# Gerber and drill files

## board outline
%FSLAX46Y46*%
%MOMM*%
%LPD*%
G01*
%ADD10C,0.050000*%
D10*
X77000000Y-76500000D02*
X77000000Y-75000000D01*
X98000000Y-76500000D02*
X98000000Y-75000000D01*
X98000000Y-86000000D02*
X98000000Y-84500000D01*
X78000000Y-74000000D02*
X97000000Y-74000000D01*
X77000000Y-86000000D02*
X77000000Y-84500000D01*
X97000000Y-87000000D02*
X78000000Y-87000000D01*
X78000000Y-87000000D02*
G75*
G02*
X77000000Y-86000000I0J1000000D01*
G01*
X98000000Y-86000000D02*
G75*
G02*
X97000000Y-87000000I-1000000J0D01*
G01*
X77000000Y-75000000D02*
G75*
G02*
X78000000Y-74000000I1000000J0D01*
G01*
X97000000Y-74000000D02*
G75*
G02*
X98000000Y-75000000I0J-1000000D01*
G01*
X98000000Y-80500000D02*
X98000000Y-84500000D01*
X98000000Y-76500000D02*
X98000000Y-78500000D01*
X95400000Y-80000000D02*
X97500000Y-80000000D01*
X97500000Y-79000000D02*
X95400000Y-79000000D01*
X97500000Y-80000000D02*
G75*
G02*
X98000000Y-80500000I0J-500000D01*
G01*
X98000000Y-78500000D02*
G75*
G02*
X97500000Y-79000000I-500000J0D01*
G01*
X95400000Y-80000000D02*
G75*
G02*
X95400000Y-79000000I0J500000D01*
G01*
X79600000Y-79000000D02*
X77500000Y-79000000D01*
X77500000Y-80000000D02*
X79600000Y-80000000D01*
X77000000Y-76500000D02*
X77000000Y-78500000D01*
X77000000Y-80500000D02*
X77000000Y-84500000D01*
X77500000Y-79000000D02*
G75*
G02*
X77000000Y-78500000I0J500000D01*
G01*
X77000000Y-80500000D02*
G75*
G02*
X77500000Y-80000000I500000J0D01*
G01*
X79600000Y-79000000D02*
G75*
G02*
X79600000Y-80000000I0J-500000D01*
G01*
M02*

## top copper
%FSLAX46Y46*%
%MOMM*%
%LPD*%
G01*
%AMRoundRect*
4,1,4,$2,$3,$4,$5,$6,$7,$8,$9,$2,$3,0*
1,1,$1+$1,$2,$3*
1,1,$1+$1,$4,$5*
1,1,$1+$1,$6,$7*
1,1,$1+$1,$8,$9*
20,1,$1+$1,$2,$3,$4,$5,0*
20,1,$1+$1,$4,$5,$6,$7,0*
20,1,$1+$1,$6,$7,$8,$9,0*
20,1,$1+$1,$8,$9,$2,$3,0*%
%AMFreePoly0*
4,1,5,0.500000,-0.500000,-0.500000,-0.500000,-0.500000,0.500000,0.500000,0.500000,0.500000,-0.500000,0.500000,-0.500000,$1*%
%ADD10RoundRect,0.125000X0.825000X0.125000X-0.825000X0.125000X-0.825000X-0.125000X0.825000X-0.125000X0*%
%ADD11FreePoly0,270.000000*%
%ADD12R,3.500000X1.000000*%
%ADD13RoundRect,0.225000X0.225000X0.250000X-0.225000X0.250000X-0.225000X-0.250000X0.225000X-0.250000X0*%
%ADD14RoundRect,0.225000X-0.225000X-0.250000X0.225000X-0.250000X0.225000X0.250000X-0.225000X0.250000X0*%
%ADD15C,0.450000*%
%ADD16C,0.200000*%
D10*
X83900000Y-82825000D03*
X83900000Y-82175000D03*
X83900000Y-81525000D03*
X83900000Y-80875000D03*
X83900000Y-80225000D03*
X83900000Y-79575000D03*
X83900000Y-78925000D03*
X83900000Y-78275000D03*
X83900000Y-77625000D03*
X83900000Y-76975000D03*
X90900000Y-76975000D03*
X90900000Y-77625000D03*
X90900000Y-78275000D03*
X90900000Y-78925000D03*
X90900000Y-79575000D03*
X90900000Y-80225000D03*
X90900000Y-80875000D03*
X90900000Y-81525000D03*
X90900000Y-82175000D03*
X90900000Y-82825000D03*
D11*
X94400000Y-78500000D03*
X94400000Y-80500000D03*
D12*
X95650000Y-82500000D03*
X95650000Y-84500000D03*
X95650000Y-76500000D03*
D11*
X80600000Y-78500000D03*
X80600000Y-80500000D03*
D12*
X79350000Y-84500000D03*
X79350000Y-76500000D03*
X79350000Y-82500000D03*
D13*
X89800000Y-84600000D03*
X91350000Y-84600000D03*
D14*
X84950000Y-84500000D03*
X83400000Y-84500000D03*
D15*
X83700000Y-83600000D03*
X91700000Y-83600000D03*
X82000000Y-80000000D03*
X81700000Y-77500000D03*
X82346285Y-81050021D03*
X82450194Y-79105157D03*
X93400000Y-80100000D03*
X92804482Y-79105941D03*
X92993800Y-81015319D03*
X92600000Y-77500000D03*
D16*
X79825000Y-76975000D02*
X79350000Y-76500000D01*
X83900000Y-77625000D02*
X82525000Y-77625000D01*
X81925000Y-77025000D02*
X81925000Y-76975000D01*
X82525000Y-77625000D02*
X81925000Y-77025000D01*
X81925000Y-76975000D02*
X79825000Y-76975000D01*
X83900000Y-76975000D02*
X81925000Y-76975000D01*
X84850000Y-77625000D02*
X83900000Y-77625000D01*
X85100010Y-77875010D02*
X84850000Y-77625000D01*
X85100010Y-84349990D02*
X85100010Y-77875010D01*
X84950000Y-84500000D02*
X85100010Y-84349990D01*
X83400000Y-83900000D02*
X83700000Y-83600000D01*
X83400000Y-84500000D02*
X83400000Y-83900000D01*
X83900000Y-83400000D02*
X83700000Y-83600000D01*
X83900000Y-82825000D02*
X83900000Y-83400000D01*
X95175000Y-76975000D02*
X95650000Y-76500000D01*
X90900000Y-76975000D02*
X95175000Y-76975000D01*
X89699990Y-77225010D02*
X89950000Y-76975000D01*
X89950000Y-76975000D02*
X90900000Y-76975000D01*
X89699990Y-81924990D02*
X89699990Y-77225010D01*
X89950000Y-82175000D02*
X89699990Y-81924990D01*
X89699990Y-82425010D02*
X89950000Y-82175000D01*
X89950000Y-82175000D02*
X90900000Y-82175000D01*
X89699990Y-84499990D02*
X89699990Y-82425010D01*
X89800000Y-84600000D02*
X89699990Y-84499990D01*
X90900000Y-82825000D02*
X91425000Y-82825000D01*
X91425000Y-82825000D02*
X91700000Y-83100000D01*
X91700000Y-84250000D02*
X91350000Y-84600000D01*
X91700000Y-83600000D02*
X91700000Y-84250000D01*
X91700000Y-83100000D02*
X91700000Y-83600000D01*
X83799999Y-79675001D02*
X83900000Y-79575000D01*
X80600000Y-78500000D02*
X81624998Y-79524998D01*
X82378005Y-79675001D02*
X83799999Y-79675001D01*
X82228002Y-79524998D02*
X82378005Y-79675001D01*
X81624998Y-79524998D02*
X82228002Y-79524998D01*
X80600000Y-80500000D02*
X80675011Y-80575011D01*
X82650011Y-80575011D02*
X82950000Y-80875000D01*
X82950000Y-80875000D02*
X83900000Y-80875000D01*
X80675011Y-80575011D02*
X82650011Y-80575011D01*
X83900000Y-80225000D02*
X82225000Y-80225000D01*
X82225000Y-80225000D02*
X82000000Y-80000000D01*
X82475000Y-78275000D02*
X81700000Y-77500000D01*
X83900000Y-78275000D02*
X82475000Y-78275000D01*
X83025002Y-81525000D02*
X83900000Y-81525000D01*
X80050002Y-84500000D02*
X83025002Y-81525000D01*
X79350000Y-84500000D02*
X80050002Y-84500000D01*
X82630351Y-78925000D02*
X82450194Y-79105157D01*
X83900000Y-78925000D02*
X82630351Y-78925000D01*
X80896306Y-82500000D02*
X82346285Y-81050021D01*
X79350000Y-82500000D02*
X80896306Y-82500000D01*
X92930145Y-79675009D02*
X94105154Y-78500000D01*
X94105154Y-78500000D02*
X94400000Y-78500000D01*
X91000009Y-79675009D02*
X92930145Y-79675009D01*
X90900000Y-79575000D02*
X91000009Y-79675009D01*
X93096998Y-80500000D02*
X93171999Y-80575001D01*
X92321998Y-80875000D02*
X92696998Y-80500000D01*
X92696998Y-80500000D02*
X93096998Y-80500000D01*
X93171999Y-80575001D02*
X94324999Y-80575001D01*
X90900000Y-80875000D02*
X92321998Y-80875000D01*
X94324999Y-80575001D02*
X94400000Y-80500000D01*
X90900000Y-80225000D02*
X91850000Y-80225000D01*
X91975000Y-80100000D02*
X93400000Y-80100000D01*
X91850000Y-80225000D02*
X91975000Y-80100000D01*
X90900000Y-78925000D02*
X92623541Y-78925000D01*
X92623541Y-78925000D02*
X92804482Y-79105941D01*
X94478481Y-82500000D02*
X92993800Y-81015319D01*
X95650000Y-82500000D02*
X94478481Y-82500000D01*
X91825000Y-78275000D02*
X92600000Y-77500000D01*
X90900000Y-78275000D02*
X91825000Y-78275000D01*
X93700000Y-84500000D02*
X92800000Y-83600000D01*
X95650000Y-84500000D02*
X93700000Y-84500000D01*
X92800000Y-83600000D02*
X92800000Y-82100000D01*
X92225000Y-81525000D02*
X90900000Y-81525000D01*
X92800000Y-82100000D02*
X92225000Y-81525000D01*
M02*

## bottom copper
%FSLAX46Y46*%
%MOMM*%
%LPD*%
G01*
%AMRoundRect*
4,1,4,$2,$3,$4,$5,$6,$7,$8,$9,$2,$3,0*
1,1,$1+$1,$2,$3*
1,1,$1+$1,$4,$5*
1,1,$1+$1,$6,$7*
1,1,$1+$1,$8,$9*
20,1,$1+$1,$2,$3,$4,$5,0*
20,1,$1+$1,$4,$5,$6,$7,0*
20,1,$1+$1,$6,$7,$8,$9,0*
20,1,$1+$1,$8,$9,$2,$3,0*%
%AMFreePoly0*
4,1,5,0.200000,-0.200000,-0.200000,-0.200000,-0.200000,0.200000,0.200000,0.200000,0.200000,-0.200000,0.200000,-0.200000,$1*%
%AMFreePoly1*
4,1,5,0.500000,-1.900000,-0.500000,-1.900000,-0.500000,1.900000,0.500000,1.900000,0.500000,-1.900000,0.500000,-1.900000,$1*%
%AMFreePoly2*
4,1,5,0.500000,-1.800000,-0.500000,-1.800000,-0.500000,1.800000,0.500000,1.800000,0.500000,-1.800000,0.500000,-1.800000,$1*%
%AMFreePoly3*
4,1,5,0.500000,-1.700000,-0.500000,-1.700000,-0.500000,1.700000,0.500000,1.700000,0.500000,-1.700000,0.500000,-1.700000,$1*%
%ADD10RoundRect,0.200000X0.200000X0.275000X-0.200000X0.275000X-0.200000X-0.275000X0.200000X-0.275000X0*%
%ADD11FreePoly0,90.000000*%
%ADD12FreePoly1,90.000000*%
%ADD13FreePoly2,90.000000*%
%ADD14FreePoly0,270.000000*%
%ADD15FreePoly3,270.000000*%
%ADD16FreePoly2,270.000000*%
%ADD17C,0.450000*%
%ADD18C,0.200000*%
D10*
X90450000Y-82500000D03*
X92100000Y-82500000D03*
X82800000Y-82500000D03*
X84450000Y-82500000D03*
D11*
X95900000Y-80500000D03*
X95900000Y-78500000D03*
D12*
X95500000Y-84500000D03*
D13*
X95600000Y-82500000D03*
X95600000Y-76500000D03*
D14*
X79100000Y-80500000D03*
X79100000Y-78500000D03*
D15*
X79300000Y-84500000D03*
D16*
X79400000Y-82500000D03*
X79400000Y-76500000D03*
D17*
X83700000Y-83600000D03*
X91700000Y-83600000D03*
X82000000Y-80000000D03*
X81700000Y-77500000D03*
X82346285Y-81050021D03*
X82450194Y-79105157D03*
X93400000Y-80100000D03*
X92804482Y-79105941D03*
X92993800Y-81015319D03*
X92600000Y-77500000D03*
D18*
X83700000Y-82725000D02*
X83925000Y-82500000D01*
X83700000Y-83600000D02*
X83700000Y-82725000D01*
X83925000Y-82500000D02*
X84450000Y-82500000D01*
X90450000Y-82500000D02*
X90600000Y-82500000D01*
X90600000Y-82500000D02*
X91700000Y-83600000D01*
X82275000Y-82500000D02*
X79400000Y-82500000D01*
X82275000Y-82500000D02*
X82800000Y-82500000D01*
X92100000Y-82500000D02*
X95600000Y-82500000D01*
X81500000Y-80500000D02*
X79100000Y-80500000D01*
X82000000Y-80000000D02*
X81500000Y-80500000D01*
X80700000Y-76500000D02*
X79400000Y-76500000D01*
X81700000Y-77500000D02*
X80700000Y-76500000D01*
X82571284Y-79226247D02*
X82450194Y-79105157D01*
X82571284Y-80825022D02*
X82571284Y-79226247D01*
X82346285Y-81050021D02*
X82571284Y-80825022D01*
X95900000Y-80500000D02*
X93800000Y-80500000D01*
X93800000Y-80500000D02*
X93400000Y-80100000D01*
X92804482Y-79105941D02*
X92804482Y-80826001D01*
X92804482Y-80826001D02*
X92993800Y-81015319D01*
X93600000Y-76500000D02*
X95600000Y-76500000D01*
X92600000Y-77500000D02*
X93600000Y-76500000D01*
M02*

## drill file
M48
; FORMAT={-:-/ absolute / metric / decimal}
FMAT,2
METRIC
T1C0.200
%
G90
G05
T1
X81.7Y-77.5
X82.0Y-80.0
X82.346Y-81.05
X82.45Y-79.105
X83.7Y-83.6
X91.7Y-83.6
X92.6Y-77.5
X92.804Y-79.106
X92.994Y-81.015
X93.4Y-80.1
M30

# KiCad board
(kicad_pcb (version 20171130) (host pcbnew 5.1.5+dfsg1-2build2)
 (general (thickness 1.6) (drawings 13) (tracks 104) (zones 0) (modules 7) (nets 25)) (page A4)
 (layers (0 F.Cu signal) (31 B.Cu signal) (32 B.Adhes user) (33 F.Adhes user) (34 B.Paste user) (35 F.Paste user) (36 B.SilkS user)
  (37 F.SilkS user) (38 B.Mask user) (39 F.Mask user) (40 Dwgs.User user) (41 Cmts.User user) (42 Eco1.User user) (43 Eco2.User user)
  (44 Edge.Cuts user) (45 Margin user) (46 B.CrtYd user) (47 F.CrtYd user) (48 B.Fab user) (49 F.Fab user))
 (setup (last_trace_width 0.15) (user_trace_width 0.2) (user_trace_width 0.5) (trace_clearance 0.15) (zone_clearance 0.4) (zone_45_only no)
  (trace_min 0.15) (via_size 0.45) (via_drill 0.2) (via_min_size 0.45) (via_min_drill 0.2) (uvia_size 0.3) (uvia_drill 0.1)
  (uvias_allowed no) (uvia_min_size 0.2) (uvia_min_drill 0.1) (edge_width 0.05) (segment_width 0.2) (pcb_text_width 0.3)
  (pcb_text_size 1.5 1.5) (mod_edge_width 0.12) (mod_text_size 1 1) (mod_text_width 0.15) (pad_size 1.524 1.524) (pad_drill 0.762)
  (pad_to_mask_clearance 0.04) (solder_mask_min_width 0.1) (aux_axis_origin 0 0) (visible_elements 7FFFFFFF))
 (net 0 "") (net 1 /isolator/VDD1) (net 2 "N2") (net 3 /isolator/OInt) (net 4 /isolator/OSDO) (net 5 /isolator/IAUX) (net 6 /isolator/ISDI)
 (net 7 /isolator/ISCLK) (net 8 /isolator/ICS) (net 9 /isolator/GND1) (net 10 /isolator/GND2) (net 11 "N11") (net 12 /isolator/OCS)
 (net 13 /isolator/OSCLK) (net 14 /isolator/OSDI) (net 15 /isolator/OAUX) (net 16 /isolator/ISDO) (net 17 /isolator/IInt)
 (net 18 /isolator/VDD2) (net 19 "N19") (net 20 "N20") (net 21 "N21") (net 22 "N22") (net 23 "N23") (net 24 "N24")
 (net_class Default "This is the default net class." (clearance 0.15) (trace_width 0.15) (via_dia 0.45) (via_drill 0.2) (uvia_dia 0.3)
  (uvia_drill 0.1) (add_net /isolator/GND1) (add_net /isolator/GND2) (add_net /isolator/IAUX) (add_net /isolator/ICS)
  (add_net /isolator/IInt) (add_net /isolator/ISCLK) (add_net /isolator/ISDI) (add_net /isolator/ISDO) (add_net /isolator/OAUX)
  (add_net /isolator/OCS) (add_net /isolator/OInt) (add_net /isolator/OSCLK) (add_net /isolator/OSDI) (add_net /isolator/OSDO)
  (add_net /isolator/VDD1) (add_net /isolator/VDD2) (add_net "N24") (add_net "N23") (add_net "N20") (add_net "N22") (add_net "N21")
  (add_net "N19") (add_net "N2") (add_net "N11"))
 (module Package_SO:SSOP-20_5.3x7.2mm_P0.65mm (layer F.Cu) (at 87.4 79.9 180)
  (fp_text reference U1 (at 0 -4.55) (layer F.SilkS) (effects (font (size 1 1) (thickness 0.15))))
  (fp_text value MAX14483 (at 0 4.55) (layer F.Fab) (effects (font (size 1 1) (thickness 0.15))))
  (pad 20 smd roundrect (at 3.5 -2.925 180) (size 1.9 0.5) (layers F.Cu F.Paste F.Mask) (roundrect_rratio 0.25) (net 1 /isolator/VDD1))
  (pad 19 smd roundrect (at 3.5 -2.275 180) (size 1.9 0.5) (layers F.Cu F.Paste F.Mask) (roundrect_rratio 0.25) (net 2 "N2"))
  (pad 18 smd roundrect (at 3.5 -1.625 180) (size 1.9 0.5) (layers F.Cu F.Paste F.Mask) (roundrect_rratio 0.25) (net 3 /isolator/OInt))
  (pad 17 smd roundrect (at 3.5 -0.975 180) (size 1.9 0.5) (layers F.Cu F.Paste F.Mask) (roundrect_rratio 0.25) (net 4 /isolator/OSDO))
  (pad 16 smd roundrect (at 3.5 -0.325 180) (size 1.9 0.5) (layers F.Cu F.Paste F.Mask) (roundrect_rratio 0.25) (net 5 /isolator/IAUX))
  (pad 15 smd roundrect (at 3.5 0.325 180) (size 1.9 0.5) (layers F.Cu F.Paste F.Mask) (roundrect_rratio 0.25) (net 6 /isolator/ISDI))
  (pad 14 smd roundrect (at 3.5 0.975 180) (size 1.9 0.5) (layers F.Cu F.Paste F.Mask) (roundrect_rratio 0.25) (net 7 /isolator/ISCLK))
  (pad 13 smd roundrect (at 3.5 1.625 180) (size 1.9 0.5) (layers F.Cu F.Paste F.Mask) (roundrect_rratio 0.25) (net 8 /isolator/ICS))
  (pad 12 smd roundrect (at 3.5 2.275 180) (size 1.9 0.5) (layers F.Cu F.Paste F.Mask) (roundrect_rratio 0.25) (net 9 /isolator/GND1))
  (pad 11 smd roundrect (at 3.5 2.925 180) (size 1.9 0.5) (layers F.Cu F.Paste F.Mask) (roundrect_rratio 0.25) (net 9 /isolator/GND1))
  (pad 10 smd roundrect (at -3.5 2.925 180) (size 1.9 0.5) (layers F.Cu F.Paste F.Mask) (roundrect_rratio 0.25) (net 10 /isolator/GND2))
  (pad 9 smd roundrect (at -3.5 2.275 180) (size 1.9 0.5) (layers F.Cu F.Paste F.Mask) (roundrect_rratio 0.25) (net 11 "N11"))
  (pad 8 smd roundrect (at -3.5 1.625 180) (size 1.9 0.5) (layers F.Cu F.Paste F.Mask) (roundrect_rratio 0.25) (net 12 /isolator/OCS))
  (pad 7 smd roundrect (at -3.5 0.975 180) (size 1.9 0.5) (layers F.Cu F.Paste F.Mask) (roundrect_rratio 0.25) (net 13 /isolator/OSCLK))
  (pad 6 smd roundrect (at -3.5 0.325 180) (size 1.9 0.5) (layers F.Cu F.Paste F.Mask) (roundrect_rratio 0.25) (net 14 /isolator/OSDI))
  (pad 5 smd roundrect (at -3.5 -0.325 180) (size 1.9 0.5) (layers F.Cu F.Paste F.Mask) (roundrect_rratio 0.25) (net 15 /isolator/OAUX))
  (pad 4 smd roundrect (at -3.5 -0.975 180) (size 1.9 0.5) (layers F.Cu F.Paste F.Mask) (roundrect_rratio 0.25) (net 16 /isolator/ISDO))
  (pad 3 smd roundrect (at -3.5 -1.625 180) (size 1.9 0.5) (layers F.Cu F.Paste F.Mask) (roundrect_rratio 0.25) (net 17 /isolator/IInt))
  (pad 2 smd roundrect (at -3.5 -2.275 180) (size 1.9 0.5) (layers F.Cu F.Paste F.Mask) (roundrect_rratio 0.25) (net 10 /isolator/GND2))
  (pad 1 smd roundrect (at -3.5 -2.925 180) (size 1.9 0.5) (layers F.Cu F.Paste F.Mask) (roundrect_rratio 0.25) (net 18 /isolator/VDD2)))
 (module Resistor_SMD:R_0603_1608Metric (layer B.Cu) (at 91.275 82.5 180)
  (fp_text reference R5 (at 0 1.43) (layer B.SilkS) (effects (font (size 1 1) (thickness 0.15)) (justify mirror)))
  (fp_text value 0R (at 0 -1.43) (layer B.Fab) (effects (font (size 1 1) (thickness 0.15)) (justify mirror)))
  (pad 2 smd roundrect (at 0.825 0 180) (size 0.8 0.95) (layers B.Cu B.Paste B.Mask) (roundrect_rratio 0.25) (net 18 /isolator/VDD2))
  (pad 1 smd roundrect (at -0.825 0 180) (size 0.8 0.95) (layers B.Cu B.Paste B.Mask) (roundrect_rratio 0.25) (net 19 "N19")))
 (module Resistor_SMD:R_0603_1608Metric (layer B.Cu) (at 83.625 82.5 180)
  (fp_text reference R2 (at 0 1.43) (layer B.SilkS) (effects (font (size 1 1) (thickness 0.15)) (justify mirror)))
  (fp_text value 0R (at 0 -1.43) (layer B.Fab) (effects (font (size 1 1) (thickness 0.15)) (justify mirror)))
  (pad 2 smd roundrect (at 0.825 0 180) (size 0.8 0.95) (layers B.Cu B.Paste B.Mask) (roundrect_rratio 0.25) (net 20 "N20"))
  (pad 1 smd roundrect (at -0.825 0 180) (size 0.8 0.95) (layers B.Cu B.Paste B.Mask) (roundrect_rratio 0.25) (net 1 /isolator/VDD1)))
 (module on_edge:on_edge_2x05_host (layer F.Cu) (at 98 80.5 270)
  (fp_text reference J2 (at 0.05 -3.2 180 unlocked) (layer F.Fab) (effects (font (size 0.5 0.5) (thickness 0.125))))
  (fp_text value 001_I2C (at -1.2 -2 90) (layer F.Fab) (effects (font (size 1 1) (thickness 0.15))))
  (fp_line (start 0 0) (end 4 0) (layer Edge.Cuts) (width 0.05))
  (fp_line (start -4 0) (end -2 0) (layer Edge.Cuts) (width 0.05))
  (fp_line (start -0.5 2.6) (end -0.5 0.5) (layer Edge.Cuts) (width 0.05))
  (fp_line (start -1.5 0.5) (end -1.5 2.6) (layer Edge.Cuts) (width 0.05))
  (fp_arc (start 0 0.5) (end 0 0) (angle -90) (layer Edge.Cuts) (width 0.05))
  (fp_arc (start -2 0.5) (end -1.5 0.5) (angle -90) (layer Edge.Cuts) (width 0.05))
  (fp_arc (start -1 2.6) (end -1.5 2.6) (angle -180) (layer Edge.Cuts) (width 0.05))
  (pad 2 smd custom (at -2 3.6 270) (size 1 1) (layers F.Cu F.Mask) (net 14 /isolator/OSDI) (zone_connect 0)
   (options (clearance outline) (anchor rect)) (primitives))
  (pad 3 smd custom (at 0 3.6 270) (size 1 1) (layers F.Cu F.Mask) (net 16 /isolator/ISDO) (zone_connect 0)
   (options (clearance outline) (anchor rect)) (primitives))
  (pad 8 smd custom (at 0 2.1 90) (size 0.4 0.4) (layers B.Cu B.Mask) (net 15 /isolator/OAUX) (zone_connect 0)
   (options (clearance outline) (anchor rect)) (primitives))
  (pad 7 smd custom (at -2 2.1 90) (size 0.4 0.4) (layers B.Cu B.Mask) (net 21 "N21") (zone_connect 0)
   (options (clearance outline) (anchor rect)) (primitives))
  (pad 4 smd rect (at 2 2.35 270) (size 1 3.5) (layers F.Cu F.Mask) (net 13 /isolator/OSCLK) (zone_connect 0))
  (pad 10 smd custom (at 4 2.5 90) (size 1 3.8) (layers B.Cu B.Mask) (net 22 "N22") (zone_connect 0)
   (options (clearance outline) (anchor rect)) (primitives))
  (pad 9 smd custom (at 2 2.4 90) (size 1 3.6) (layers B.Cu B.Mask) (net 19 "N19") (zone_connect 0)
   (options (clearance outline) (anchor rect)) (primitives))
  (pad 6 smd custom (at -4 2.4 90) (size 1 3.6) (layers B.Cu B.Mask) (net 12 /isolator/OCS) (zone_connect 0)
   (options (clearance outline) (anchor rect)) (primitives))
  (pad 5 smd rect (at 4 2.35 270) (size 1 3.5) (layers F.Cu F.Mask) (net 17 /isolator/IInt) (zone_connect 0))
  (pad 1 smd rect (at -4 2.35 270) (size 1 3.5) (layers F.Cu F.Mask) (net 10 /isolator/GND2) (zone_connect 0)))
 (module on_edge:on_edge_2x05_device (layer F.Cu) (at 77 80.5 270)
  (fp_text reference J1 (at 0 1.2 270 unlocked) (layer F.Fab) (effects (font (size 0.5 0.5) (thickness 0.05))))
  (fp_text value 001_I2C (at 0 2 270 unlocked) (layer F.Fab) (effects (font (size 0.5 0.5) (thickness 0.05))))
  (fp_line (start -1.5 -2.6) (end -1.5 -0.5) (layer Edge.Cuts) (width 0.05))
  (fp_line (start -0.5 -0.5) (end -0.5 -2.6) (layer Edge.Cuts) (width 0.05))
  (fp_line (start -4 0) (end -2 0) (layer Edge.Cuts) (width 0.05))
  (fp_line (start 0 0) (end 4 0) (layer Edge.Cuts) (width 0.05))
  (fp_arc (start -2 -0.5) (end -2 0) (angle -90) (layer Edge.Cuts) (width 0.05))
  (fp_arc (start 0 -0.5) (end -0.5 -0.5) (angle -90) (layer Edge.Cuts) (width 0.05))
  (fp_arc (start -1 -2.6) (end -0.5 -2.6) (angle -180) (layer Edge.Cuts) (width 0.05))
  (pad 2 smd custom (at -2 -3.6 270) (size 1 1) (layers F.Cu F.Mask) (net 6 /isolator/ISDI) (zone_connect 0)
   (options (clearance outline) (anchor rect)) (primitives))
  (pad 3 smd custom (at 0 -3.6 270) (size 1 1) (layers F.Cu F.Mask) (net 4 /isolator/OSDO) (zone_connect 0)
   (options (clearance outline) (anchor rect)) (primitives))
  (pad 8 smd custom (at 0 -2.1 270) (size 0.4 0.4) (layers B.Cu B.Mask) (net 5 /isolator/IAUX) (zone_connect 0)
   (options (clearance outline) (anchor rect)) (primitives))
  (pad 7 smd custom (at -2 -2.1 270) (size 0.4 0.4) (layers B.Cu B.Mask) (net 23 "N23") (zone_connect 0)
   (options (clearance outline) (anchor rect)) (primitives))
  (pad 10 smd custom (at 4 -2.3 270) (size 1 3.4) (layers B.Cu B.Mask) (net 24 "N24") (zone_connect 0)
   (options (clearance outline) (anchor rect)) (primitives))
  (pad 9 smd custom (at 2 -2.4 270) (size 1 3.6) (layers B.Cu B.Mask) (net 20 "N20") (zone_connect 0)
   (options (clearance outline) (anchor rect)) (primitives))
  (pad 6 smd custom (at -4 -2.4 270) (size 1 3.6) (layers B.Cu B.Mask) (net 8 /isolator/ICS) (zone_connect 0)
   (options (clearance outline) (anchor rect)) (primitives))
  (pad 5 smd rect (at 4 -2.35 90) (size 1 3.5) (layers F.Cu F.Mask) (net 3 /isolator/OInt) (zone_connect 0))
  (pad 1 smd rect (at -4 -2.35 90) (size 1 3.5) (layers F.Cu F.Mask) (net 9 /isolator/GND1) (zone_connect 0))
  (pad 4 smd rect (at 2 -2.35 90) (size 1 3.5) (layers F.Cu F.Mask) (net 7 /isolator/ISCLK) (zone_connect 0)))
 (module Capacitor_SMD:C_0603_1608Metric (layer F.Cu) (at 90.575 84.6 180)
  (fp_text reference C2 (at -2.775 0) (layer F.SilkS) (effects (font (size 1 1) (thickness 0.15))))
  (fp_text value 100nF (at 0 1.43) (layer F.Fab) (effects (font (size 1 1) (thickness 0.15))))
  (pad 2 smd roundrect (at 0.775 0 180) (size 0.9 0.95) (layers F.Cu F.Paste F.Mask) (roundrect_rratio 0.25) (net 10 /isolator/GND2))
  (pad 1 smd roundrect (at -0.775 0 180) (size 0.9 0.95) (layers F.Cu F.Paste F.Mask) (roundrect_rratio 0.25) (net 18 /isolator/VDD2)))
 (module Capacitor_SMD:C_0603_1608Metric (layer F.Cu) (at 84.175 84.5)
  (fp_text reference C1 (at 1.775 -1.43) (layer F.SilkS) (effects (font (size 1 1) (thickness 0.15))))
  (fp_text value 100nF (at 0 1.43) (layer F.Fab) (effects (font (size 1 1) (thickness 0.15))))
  (pad 2 smd roundrect (at 0.775 0) (size 0.9 0.95) (layers F.Cu F.Paste F.Mask) (roundrect_rratio 0.25) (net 9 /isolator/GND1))
  (pad 1 smd roundrect (at -0.775 0) (size 0.9 0.95) (layers F.Cu F.Paste F.Mask) (roundrect_rratio 0.25) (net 1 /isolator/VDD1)))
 (gr_line (start 77 76.5) (end 77 75) (layer Edge.Cuts) (width 0.05))
 (gr_line (start 98 76.5) (end 98 75) (layer Edge.Cuts) (width 0.05))
 (gr_line (start 98 86) (end 98 84.5) (layer Edge.Cuts) (width 0.05))
 (gr_line (start 78 74) (end 97 74) (layer Edge.Cuts) (width 0.05))
 (gr_line (start 77 86) (end 77 84.5) (layer Edge.Cuts) (width 0.05))
 (gr_line (start 97 87) (end 78 87) (layer Edge.Cuts) (width 0.05))
 (gr_arc (start 78 86) (end 77 86) (angle -90) (layer Edge.Cuts) (width 0.05))
 (gr_arc (start 97 86) (end 97 87) (angle -90) (layer Edge.Cuts) (width 0.05))
 (gr_arc (start 78 75) (end 78 74) (angle -90) (layer Edge.Cuts) (width 0.05))
 (gr_arc (start 97 75) (end 98 75) (angle -90) (layer Edge.Cuts) (width 0.05))
 (segment (start 79.825 76.975) (end 79.35 76.5) (width 0.2) (layer F.Cu) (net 9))
 (segment (start 83.9 77.625) (end 82.525 77.625) (width 0.2) (layer F.Cu) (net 9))
 (segment (start 81.925 77.025) (end 81.925 76.975) (width 0.2) (layer F.Cu) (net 9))
 (segment (start 82.525 77.625) (end 81.925 77.025) (width 0.2) (layer F.Cu) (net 9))
 (segment (start 81.925 76.975) (end 79.825 76.975) (width 0.2) (layer F.Cu) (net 9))
 (segment (start 83.9 76.975) (end 81.925 76.975) (width 0.2) (layer F.Cu) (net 9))
 (segment (start 84.85 77.625) (end 83.9 77.625) (width 0.2) (layer F.Cu) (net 9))
 (segment (start 85.10001 77.87501) (end 84.85 77.625) (width 0.2) (layer F.Cu) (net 9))
 (segment (start 85.10001 84.34999) (end 85.10001 77.87501) (width 0.2) (layer F.Cu) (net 9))
 (segment (start 84.95 84.5) (end 85.10001 84.34999) (width 0.2) (layer F.Cu) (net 9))
 (via (at 83.7 83.6) (size 0.45) (drill 0.2) (layers F.Cu B.Cu) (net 1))
 (segment (start 83.4 83.9) (end 83.7 83.6) (width 0.2) (layer F.Cu) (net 1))
 (segment (start 83.4 84.5) (end 83.4 83.9) (width 0.2) (layer F.Cu) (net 1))
 (segment (start 83.7 82.725) (end 83.925 82.5) (width 0.2) (layer B.Cu) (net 1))
 (segment (start 83.7 83.6) (end 83.7 82.725) (width 0.2) (layer B.Cu) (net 1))
 (segment (start 83.9 83.4) (end 83.7 83.6) (width 0.2) (layer F.Cu) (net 1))
 (segment (start 83.9 82.825) (end 83.9 83.4) (width 0.2) (layer F.Cu) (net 1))
 (segment (start 83.925 82.5) (end 84.45 82.5) (width 0.2) (layer B.Cu) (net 1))
 (segment (start 95.175 76.975) (end 95.65 76.5) (width 0.2) (layer F.Cu) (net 10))
 (segment (start 90.9 76.975) (end 95.175 76.975) (width 0.2) (layer F.Cu) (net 10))
 (segment (start 89.69999 77.22501) (end 89.95 76.975) (width 0.2) (layer F.Cu) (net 10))
 (segment (start 89.95 76.975) (end 90.9 76.975) (width 0.2) (layer F.Cu) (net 10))
 (segment (start 89.69999 81.92499) (end 89.69999 77.22501) (width 0.2) (layer F.Cu) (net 10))
 (segment (start 89.95 82.175) (end 89.69999 81.92499) (width 0.2) (layer F.Cu) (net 10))
 (segment (start 89.69999 82.42501) (end 89.95 82.175) (width 0.2) (layer F.Cu) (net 10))
 (segment (start 89.95 82.175) (end 90.9 82.175) (width 0.2) (layer F.Cu) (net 10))
 (segment (start 89.69999 84.49999) (end 89.69999 82.42501) (width 0.2) (layer F.Cu) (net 10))
 (segment (start 89.8 84.6) (end 89.69999 84.49999) (width 0.2) (layer F.Cu) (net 10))
 (segment (start 90.9 82.825) (end 91.425 82.825) (width 0.2) (layer F.Cu) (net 18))
 (segment (start 91.425 82.825) (end 91.7 83.1) (width 0.2) (layer F.Cu) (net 18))
 (segment (start 91.7 84.25) (end 91.35 84.6) (width 0.2) (layer F.Cu) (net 18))
 (via (at 91.7 83.6) (size 0.45) (drill 0.2) (layers F.Cu B.Cu) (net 18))
 (segment (start 90.45 82.5) (end 90.6 82.5) (width 0.2) (layer B.Cu) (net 18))
 (segment (start 91.7 83.6) (end 91.7 84.25) (width 0.2) (layer F.Cu) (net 18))
 (segment (start 90.6 82.5) (end 91.7 83.6) (width 0.2) (layer B.Cu) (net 18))
 (segment (start 91.7 83.1) (end 91.7 83.6) (width 0.2) (layer F.Cu) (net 18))
 (segment (start 82.275 82.5) (end 79.4 82.5) (width 0.2) (layer B.Cu) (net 20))
 (segment (start 82.275 82.5) (end 82.8 82.5) (width 0.2) (layer B.Cu) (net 20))
 (segment (start 92.1 82.5) (end 95.6 82.5) (width 0.2) (layer B.Cu) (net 19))
 (segment (start 83.799999 79.675001) (end 83.9 79.575) (width 0.2) (layer F.Cu) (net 6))
 (segment (start 80.6 78.5) (end 81.624998 79.524998) (width 0.2) (layer F.Cu) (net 6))
 (segment (start 82.378005 79.675001) (end 83.799999 79.675001) (width 0.2) (layer F.Cu) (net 6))
 (segment (start 82.228002 79.524998) (end 82.378005 79.675001) (width 0.2) (layer F.Cu) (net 6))
 (segment (start 81.624998 79.524998) (end 82.228002 79.524998) (width 0.2) (layer F.Cu) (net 6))
 (segment (start 80.6 80.5) (end 80.675011 80.575011) (width 0.2) (layer F.Cu) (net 4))
 (segment (start 82.650011 80.575011) (end 82.95 80.875) (width 0.2) (layer F.Cu) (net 4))
 (segment (start 82.95 80.875) (end 83.9 80.875) (width 0.2) (layer F.Cu) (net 4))
 (segment (start 80.675011 80.575011) (end 82.650011 80.575011) (width 0.2) (layer F.Cu) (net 4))
 (segment (start 83.9 80.225) (end 82.225 80.225) (width 0.2) (layer F.Cu) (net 5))
 (via (at 82 80) (size 0.45) (drill 0.2) (layers F.Cu B.Cu) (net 5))
 (segment (start 82.225 80.225) (end 82 80) (width 0.2) (layer F.Cu) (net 5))
 (segment (start 81.5 80.5) (end 79.1 80.5) (width 0.2) (layer B.Cu) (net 5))
 (segment (start 82 80) (end 81.5 80.5) (width 0.2) (layer B.Cu) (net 5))
 (via (at 81.7 77.5) (size 0.45) (drill 0.2) (layers F.Cu B.Cu) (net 8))
 (segment (start 82.475 78.275) (end 81.7 77.5) (width 0.2) (layer F.Cu) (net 8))
 (segment (start 83.9 78.275) (end 82.475 78.275) (width 0.2) (layer F.Cu) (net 8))
 (segment (start 80.7 76.5) (end 79.4 76.5) (width 0.2) (layer B.Cu) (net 8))
 (segment (start 81.7 77.5) (end 80.7 76.5) (width 0.2) (layer B.Cu) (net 8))
 (segment (start 83.025002 81.525) (end 83.9 81.525) (width 0.2) (layer F.Cu) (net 3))
 (segment (start 80.050002 84.5) (end 83.025002 81.525) (width 0.2) (layer F.Cu) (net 3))
 (segment (start 79.35 84.5) (end 80.050002 84.5) (width 0.2) (layer F.Cu) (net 3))
 (via (at 82.346285 81.050021) (size 0.45) (drill 0.2) (layers F.Cu B.Cu) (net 7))
 (segment (start 82.571284 79.226247) (end 82.450194 79.105157) (width 0.2) (layer B.Cu) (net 7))
 (segment (start 82.571284 80.825022) (end 82.571284 79.226247) (width 0.2) (layer B.Cu) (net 7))
 (segment (start 82.346285 81.050021) (end 82.571284 80.825022) (width 0.2) (layer B.Cu) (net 7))
 (segment (start 82.630351 78.925) (end 82.450194 79.105157) (width 0.2) (layer F.Cu) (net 7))
 (segment (start 83.9 78.925) (end 82.630351 78.925) (width 0.2) (layer F.Cu) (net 7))
 (via (at 82.450194 79.105157) (size 0.45) (drill 0.2) (layers F.Cu B.Cu) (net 7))
 (segment (start 80.896306 82.5) (end 82.346285 81.050021) (width 0.2) (layer F.Cu) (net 7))
 (segment (start 79.35 82.5) (end 80.896306 82.5) (width 0.2) (layer F.Cu) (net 7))
 (segment (start 92.930145 79.675009) (end 94.105154 78.5) (width 0.2) (layer F.Cu) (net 14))
 (segment (start 94.105154 78.5) (end 94.4 78.5) (width 0.2) (layer F.Cu) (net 14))
 (segment (start 91.000009 79.675009) (end 92.930145 79.675009) (width 0.2) (layer F.Cu) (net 14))
 (segment (start 90.9 79.575) (end 91.000009 79.675009) (width 0.2) (layer F.Cu) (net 14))
 (segment (start 93.096998 80.5) (end 93.171999 80.575001) (width 0.2) (layer F.Cu) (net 16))
 (segment (start 92.321998 80.875) (end 92.696998 80.5) (width 0.2) (layer F.Cu) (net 16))
 (segment (start 92.696998 80.5) (end 93.096998 80.5) (width 0.2) (layer F.Cu) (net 16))
 (segment (start 93.171999 80.575001) (end 94.324999 80.575001) (width 0.2) (layer F.Cu) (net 16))
 (segment (start 90.9 80.875) (end 92.321998 80.875) (width 0.2) (layer F.Cu) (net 16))
 (segment (start 94.324999 80.575001) (end 94.4 80.5) (width 0.2) (layer F.Cu) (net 16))
 (via (at 93.4 80.1) (size 0.45) (drill 0.2) (layers F.Cu B.Cu) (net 15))
 (segment (start 95.9 80.5) (end 93.8 80.5) (width 0.2) (layer B.Cu) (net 15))
 (segment (start 90.9 80.225) (end 91.85 80.225) (width 0.2) (layer F.Cu) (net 15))
 (segment (start 93.8 80.5) (end 93.4 80.1) (width 0.2) (layer B.Cu) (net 15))
 (segment (start 91.975 80.1) (end 93.4 80.1) (width 0.2) (layer F.Cu) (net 15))
 (segment (start 91.85 80.225) (end 91.975 80.1) (width 0.2) (layer F.Cu) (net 15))
 (via (at 92.804482 79.105941) (size 0.45) (drill 0.2) (layers F.Cu B.Cu) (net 13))
 (segment (start 90.9 78.925) (end 92.623541 78.925) (width 0.2) (layer F.Cu) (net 13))
 (segment (start 92.623541 78.925) (end 92.804482 79.105941) (width 0.2) (layer F.Cu) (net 13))
 (segment (start 94.478481 82.5) (end 92.9938 81.015319) (width 0.2) (layer F.Cu) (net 13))
 (segment (start 92.804482 79.105941) (end 92.804482 80.826001) (width 0.2) (layer B.Cu) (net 13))
 (via (at 92.9938 81.015319) (size 0.45) (drill 0.2) (layers F.Cu B.Cu) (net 13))
 (segment (start 92.804482 80.826001) (end 92.9938 81.015319) (width 0.2) (layer B.Cu) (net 13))
 (segment (start 95.65 82.5) (end 94.478481 82.5) (width 0.2) (layer F.Cu) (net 13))
 (via (at 92.6 77.5) (size 0.45) (drill 0.2) (layers F.Cu B.Cu) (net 12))
 (segment (start 91.825 78.275) (end 92.6 77.5) (width 0.2) (layer F.Cu) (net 12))
 (segment (start 90.9 78.275) (end 91.825 78.275) (width 0.2) (layer F.Cu) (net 12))
 (segment (start 93.6 76.5) (end 95.6 76.5) (width 0.2) (layer B.Cu) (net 12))
 (segment (start 92.6 77.5) (end 93.6 76.5) (width 0.2) (layer B.Cu) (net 12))
 (segment (start 93.7 84.5) (end 92.8 83.6) (width 0.2) (layer F.Cu) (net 17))
 (segment (start 95.65 84.5) (end 93.7 84.5) (width 0.2) (layer F.Cu) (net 17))
 (segment (start 92.8 83.6) (end 92.8 82.1) (width 0.2) (layer F.Cu) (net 17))
 (segment (start 92.225 81.525) (end 90.9 81.525) (width 0.2) (layer F.Cu) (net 17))
 (segment (start 92.8 82.1) (end 92.225 81.525) (width 0.2) (layer F.Cu) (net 17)))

